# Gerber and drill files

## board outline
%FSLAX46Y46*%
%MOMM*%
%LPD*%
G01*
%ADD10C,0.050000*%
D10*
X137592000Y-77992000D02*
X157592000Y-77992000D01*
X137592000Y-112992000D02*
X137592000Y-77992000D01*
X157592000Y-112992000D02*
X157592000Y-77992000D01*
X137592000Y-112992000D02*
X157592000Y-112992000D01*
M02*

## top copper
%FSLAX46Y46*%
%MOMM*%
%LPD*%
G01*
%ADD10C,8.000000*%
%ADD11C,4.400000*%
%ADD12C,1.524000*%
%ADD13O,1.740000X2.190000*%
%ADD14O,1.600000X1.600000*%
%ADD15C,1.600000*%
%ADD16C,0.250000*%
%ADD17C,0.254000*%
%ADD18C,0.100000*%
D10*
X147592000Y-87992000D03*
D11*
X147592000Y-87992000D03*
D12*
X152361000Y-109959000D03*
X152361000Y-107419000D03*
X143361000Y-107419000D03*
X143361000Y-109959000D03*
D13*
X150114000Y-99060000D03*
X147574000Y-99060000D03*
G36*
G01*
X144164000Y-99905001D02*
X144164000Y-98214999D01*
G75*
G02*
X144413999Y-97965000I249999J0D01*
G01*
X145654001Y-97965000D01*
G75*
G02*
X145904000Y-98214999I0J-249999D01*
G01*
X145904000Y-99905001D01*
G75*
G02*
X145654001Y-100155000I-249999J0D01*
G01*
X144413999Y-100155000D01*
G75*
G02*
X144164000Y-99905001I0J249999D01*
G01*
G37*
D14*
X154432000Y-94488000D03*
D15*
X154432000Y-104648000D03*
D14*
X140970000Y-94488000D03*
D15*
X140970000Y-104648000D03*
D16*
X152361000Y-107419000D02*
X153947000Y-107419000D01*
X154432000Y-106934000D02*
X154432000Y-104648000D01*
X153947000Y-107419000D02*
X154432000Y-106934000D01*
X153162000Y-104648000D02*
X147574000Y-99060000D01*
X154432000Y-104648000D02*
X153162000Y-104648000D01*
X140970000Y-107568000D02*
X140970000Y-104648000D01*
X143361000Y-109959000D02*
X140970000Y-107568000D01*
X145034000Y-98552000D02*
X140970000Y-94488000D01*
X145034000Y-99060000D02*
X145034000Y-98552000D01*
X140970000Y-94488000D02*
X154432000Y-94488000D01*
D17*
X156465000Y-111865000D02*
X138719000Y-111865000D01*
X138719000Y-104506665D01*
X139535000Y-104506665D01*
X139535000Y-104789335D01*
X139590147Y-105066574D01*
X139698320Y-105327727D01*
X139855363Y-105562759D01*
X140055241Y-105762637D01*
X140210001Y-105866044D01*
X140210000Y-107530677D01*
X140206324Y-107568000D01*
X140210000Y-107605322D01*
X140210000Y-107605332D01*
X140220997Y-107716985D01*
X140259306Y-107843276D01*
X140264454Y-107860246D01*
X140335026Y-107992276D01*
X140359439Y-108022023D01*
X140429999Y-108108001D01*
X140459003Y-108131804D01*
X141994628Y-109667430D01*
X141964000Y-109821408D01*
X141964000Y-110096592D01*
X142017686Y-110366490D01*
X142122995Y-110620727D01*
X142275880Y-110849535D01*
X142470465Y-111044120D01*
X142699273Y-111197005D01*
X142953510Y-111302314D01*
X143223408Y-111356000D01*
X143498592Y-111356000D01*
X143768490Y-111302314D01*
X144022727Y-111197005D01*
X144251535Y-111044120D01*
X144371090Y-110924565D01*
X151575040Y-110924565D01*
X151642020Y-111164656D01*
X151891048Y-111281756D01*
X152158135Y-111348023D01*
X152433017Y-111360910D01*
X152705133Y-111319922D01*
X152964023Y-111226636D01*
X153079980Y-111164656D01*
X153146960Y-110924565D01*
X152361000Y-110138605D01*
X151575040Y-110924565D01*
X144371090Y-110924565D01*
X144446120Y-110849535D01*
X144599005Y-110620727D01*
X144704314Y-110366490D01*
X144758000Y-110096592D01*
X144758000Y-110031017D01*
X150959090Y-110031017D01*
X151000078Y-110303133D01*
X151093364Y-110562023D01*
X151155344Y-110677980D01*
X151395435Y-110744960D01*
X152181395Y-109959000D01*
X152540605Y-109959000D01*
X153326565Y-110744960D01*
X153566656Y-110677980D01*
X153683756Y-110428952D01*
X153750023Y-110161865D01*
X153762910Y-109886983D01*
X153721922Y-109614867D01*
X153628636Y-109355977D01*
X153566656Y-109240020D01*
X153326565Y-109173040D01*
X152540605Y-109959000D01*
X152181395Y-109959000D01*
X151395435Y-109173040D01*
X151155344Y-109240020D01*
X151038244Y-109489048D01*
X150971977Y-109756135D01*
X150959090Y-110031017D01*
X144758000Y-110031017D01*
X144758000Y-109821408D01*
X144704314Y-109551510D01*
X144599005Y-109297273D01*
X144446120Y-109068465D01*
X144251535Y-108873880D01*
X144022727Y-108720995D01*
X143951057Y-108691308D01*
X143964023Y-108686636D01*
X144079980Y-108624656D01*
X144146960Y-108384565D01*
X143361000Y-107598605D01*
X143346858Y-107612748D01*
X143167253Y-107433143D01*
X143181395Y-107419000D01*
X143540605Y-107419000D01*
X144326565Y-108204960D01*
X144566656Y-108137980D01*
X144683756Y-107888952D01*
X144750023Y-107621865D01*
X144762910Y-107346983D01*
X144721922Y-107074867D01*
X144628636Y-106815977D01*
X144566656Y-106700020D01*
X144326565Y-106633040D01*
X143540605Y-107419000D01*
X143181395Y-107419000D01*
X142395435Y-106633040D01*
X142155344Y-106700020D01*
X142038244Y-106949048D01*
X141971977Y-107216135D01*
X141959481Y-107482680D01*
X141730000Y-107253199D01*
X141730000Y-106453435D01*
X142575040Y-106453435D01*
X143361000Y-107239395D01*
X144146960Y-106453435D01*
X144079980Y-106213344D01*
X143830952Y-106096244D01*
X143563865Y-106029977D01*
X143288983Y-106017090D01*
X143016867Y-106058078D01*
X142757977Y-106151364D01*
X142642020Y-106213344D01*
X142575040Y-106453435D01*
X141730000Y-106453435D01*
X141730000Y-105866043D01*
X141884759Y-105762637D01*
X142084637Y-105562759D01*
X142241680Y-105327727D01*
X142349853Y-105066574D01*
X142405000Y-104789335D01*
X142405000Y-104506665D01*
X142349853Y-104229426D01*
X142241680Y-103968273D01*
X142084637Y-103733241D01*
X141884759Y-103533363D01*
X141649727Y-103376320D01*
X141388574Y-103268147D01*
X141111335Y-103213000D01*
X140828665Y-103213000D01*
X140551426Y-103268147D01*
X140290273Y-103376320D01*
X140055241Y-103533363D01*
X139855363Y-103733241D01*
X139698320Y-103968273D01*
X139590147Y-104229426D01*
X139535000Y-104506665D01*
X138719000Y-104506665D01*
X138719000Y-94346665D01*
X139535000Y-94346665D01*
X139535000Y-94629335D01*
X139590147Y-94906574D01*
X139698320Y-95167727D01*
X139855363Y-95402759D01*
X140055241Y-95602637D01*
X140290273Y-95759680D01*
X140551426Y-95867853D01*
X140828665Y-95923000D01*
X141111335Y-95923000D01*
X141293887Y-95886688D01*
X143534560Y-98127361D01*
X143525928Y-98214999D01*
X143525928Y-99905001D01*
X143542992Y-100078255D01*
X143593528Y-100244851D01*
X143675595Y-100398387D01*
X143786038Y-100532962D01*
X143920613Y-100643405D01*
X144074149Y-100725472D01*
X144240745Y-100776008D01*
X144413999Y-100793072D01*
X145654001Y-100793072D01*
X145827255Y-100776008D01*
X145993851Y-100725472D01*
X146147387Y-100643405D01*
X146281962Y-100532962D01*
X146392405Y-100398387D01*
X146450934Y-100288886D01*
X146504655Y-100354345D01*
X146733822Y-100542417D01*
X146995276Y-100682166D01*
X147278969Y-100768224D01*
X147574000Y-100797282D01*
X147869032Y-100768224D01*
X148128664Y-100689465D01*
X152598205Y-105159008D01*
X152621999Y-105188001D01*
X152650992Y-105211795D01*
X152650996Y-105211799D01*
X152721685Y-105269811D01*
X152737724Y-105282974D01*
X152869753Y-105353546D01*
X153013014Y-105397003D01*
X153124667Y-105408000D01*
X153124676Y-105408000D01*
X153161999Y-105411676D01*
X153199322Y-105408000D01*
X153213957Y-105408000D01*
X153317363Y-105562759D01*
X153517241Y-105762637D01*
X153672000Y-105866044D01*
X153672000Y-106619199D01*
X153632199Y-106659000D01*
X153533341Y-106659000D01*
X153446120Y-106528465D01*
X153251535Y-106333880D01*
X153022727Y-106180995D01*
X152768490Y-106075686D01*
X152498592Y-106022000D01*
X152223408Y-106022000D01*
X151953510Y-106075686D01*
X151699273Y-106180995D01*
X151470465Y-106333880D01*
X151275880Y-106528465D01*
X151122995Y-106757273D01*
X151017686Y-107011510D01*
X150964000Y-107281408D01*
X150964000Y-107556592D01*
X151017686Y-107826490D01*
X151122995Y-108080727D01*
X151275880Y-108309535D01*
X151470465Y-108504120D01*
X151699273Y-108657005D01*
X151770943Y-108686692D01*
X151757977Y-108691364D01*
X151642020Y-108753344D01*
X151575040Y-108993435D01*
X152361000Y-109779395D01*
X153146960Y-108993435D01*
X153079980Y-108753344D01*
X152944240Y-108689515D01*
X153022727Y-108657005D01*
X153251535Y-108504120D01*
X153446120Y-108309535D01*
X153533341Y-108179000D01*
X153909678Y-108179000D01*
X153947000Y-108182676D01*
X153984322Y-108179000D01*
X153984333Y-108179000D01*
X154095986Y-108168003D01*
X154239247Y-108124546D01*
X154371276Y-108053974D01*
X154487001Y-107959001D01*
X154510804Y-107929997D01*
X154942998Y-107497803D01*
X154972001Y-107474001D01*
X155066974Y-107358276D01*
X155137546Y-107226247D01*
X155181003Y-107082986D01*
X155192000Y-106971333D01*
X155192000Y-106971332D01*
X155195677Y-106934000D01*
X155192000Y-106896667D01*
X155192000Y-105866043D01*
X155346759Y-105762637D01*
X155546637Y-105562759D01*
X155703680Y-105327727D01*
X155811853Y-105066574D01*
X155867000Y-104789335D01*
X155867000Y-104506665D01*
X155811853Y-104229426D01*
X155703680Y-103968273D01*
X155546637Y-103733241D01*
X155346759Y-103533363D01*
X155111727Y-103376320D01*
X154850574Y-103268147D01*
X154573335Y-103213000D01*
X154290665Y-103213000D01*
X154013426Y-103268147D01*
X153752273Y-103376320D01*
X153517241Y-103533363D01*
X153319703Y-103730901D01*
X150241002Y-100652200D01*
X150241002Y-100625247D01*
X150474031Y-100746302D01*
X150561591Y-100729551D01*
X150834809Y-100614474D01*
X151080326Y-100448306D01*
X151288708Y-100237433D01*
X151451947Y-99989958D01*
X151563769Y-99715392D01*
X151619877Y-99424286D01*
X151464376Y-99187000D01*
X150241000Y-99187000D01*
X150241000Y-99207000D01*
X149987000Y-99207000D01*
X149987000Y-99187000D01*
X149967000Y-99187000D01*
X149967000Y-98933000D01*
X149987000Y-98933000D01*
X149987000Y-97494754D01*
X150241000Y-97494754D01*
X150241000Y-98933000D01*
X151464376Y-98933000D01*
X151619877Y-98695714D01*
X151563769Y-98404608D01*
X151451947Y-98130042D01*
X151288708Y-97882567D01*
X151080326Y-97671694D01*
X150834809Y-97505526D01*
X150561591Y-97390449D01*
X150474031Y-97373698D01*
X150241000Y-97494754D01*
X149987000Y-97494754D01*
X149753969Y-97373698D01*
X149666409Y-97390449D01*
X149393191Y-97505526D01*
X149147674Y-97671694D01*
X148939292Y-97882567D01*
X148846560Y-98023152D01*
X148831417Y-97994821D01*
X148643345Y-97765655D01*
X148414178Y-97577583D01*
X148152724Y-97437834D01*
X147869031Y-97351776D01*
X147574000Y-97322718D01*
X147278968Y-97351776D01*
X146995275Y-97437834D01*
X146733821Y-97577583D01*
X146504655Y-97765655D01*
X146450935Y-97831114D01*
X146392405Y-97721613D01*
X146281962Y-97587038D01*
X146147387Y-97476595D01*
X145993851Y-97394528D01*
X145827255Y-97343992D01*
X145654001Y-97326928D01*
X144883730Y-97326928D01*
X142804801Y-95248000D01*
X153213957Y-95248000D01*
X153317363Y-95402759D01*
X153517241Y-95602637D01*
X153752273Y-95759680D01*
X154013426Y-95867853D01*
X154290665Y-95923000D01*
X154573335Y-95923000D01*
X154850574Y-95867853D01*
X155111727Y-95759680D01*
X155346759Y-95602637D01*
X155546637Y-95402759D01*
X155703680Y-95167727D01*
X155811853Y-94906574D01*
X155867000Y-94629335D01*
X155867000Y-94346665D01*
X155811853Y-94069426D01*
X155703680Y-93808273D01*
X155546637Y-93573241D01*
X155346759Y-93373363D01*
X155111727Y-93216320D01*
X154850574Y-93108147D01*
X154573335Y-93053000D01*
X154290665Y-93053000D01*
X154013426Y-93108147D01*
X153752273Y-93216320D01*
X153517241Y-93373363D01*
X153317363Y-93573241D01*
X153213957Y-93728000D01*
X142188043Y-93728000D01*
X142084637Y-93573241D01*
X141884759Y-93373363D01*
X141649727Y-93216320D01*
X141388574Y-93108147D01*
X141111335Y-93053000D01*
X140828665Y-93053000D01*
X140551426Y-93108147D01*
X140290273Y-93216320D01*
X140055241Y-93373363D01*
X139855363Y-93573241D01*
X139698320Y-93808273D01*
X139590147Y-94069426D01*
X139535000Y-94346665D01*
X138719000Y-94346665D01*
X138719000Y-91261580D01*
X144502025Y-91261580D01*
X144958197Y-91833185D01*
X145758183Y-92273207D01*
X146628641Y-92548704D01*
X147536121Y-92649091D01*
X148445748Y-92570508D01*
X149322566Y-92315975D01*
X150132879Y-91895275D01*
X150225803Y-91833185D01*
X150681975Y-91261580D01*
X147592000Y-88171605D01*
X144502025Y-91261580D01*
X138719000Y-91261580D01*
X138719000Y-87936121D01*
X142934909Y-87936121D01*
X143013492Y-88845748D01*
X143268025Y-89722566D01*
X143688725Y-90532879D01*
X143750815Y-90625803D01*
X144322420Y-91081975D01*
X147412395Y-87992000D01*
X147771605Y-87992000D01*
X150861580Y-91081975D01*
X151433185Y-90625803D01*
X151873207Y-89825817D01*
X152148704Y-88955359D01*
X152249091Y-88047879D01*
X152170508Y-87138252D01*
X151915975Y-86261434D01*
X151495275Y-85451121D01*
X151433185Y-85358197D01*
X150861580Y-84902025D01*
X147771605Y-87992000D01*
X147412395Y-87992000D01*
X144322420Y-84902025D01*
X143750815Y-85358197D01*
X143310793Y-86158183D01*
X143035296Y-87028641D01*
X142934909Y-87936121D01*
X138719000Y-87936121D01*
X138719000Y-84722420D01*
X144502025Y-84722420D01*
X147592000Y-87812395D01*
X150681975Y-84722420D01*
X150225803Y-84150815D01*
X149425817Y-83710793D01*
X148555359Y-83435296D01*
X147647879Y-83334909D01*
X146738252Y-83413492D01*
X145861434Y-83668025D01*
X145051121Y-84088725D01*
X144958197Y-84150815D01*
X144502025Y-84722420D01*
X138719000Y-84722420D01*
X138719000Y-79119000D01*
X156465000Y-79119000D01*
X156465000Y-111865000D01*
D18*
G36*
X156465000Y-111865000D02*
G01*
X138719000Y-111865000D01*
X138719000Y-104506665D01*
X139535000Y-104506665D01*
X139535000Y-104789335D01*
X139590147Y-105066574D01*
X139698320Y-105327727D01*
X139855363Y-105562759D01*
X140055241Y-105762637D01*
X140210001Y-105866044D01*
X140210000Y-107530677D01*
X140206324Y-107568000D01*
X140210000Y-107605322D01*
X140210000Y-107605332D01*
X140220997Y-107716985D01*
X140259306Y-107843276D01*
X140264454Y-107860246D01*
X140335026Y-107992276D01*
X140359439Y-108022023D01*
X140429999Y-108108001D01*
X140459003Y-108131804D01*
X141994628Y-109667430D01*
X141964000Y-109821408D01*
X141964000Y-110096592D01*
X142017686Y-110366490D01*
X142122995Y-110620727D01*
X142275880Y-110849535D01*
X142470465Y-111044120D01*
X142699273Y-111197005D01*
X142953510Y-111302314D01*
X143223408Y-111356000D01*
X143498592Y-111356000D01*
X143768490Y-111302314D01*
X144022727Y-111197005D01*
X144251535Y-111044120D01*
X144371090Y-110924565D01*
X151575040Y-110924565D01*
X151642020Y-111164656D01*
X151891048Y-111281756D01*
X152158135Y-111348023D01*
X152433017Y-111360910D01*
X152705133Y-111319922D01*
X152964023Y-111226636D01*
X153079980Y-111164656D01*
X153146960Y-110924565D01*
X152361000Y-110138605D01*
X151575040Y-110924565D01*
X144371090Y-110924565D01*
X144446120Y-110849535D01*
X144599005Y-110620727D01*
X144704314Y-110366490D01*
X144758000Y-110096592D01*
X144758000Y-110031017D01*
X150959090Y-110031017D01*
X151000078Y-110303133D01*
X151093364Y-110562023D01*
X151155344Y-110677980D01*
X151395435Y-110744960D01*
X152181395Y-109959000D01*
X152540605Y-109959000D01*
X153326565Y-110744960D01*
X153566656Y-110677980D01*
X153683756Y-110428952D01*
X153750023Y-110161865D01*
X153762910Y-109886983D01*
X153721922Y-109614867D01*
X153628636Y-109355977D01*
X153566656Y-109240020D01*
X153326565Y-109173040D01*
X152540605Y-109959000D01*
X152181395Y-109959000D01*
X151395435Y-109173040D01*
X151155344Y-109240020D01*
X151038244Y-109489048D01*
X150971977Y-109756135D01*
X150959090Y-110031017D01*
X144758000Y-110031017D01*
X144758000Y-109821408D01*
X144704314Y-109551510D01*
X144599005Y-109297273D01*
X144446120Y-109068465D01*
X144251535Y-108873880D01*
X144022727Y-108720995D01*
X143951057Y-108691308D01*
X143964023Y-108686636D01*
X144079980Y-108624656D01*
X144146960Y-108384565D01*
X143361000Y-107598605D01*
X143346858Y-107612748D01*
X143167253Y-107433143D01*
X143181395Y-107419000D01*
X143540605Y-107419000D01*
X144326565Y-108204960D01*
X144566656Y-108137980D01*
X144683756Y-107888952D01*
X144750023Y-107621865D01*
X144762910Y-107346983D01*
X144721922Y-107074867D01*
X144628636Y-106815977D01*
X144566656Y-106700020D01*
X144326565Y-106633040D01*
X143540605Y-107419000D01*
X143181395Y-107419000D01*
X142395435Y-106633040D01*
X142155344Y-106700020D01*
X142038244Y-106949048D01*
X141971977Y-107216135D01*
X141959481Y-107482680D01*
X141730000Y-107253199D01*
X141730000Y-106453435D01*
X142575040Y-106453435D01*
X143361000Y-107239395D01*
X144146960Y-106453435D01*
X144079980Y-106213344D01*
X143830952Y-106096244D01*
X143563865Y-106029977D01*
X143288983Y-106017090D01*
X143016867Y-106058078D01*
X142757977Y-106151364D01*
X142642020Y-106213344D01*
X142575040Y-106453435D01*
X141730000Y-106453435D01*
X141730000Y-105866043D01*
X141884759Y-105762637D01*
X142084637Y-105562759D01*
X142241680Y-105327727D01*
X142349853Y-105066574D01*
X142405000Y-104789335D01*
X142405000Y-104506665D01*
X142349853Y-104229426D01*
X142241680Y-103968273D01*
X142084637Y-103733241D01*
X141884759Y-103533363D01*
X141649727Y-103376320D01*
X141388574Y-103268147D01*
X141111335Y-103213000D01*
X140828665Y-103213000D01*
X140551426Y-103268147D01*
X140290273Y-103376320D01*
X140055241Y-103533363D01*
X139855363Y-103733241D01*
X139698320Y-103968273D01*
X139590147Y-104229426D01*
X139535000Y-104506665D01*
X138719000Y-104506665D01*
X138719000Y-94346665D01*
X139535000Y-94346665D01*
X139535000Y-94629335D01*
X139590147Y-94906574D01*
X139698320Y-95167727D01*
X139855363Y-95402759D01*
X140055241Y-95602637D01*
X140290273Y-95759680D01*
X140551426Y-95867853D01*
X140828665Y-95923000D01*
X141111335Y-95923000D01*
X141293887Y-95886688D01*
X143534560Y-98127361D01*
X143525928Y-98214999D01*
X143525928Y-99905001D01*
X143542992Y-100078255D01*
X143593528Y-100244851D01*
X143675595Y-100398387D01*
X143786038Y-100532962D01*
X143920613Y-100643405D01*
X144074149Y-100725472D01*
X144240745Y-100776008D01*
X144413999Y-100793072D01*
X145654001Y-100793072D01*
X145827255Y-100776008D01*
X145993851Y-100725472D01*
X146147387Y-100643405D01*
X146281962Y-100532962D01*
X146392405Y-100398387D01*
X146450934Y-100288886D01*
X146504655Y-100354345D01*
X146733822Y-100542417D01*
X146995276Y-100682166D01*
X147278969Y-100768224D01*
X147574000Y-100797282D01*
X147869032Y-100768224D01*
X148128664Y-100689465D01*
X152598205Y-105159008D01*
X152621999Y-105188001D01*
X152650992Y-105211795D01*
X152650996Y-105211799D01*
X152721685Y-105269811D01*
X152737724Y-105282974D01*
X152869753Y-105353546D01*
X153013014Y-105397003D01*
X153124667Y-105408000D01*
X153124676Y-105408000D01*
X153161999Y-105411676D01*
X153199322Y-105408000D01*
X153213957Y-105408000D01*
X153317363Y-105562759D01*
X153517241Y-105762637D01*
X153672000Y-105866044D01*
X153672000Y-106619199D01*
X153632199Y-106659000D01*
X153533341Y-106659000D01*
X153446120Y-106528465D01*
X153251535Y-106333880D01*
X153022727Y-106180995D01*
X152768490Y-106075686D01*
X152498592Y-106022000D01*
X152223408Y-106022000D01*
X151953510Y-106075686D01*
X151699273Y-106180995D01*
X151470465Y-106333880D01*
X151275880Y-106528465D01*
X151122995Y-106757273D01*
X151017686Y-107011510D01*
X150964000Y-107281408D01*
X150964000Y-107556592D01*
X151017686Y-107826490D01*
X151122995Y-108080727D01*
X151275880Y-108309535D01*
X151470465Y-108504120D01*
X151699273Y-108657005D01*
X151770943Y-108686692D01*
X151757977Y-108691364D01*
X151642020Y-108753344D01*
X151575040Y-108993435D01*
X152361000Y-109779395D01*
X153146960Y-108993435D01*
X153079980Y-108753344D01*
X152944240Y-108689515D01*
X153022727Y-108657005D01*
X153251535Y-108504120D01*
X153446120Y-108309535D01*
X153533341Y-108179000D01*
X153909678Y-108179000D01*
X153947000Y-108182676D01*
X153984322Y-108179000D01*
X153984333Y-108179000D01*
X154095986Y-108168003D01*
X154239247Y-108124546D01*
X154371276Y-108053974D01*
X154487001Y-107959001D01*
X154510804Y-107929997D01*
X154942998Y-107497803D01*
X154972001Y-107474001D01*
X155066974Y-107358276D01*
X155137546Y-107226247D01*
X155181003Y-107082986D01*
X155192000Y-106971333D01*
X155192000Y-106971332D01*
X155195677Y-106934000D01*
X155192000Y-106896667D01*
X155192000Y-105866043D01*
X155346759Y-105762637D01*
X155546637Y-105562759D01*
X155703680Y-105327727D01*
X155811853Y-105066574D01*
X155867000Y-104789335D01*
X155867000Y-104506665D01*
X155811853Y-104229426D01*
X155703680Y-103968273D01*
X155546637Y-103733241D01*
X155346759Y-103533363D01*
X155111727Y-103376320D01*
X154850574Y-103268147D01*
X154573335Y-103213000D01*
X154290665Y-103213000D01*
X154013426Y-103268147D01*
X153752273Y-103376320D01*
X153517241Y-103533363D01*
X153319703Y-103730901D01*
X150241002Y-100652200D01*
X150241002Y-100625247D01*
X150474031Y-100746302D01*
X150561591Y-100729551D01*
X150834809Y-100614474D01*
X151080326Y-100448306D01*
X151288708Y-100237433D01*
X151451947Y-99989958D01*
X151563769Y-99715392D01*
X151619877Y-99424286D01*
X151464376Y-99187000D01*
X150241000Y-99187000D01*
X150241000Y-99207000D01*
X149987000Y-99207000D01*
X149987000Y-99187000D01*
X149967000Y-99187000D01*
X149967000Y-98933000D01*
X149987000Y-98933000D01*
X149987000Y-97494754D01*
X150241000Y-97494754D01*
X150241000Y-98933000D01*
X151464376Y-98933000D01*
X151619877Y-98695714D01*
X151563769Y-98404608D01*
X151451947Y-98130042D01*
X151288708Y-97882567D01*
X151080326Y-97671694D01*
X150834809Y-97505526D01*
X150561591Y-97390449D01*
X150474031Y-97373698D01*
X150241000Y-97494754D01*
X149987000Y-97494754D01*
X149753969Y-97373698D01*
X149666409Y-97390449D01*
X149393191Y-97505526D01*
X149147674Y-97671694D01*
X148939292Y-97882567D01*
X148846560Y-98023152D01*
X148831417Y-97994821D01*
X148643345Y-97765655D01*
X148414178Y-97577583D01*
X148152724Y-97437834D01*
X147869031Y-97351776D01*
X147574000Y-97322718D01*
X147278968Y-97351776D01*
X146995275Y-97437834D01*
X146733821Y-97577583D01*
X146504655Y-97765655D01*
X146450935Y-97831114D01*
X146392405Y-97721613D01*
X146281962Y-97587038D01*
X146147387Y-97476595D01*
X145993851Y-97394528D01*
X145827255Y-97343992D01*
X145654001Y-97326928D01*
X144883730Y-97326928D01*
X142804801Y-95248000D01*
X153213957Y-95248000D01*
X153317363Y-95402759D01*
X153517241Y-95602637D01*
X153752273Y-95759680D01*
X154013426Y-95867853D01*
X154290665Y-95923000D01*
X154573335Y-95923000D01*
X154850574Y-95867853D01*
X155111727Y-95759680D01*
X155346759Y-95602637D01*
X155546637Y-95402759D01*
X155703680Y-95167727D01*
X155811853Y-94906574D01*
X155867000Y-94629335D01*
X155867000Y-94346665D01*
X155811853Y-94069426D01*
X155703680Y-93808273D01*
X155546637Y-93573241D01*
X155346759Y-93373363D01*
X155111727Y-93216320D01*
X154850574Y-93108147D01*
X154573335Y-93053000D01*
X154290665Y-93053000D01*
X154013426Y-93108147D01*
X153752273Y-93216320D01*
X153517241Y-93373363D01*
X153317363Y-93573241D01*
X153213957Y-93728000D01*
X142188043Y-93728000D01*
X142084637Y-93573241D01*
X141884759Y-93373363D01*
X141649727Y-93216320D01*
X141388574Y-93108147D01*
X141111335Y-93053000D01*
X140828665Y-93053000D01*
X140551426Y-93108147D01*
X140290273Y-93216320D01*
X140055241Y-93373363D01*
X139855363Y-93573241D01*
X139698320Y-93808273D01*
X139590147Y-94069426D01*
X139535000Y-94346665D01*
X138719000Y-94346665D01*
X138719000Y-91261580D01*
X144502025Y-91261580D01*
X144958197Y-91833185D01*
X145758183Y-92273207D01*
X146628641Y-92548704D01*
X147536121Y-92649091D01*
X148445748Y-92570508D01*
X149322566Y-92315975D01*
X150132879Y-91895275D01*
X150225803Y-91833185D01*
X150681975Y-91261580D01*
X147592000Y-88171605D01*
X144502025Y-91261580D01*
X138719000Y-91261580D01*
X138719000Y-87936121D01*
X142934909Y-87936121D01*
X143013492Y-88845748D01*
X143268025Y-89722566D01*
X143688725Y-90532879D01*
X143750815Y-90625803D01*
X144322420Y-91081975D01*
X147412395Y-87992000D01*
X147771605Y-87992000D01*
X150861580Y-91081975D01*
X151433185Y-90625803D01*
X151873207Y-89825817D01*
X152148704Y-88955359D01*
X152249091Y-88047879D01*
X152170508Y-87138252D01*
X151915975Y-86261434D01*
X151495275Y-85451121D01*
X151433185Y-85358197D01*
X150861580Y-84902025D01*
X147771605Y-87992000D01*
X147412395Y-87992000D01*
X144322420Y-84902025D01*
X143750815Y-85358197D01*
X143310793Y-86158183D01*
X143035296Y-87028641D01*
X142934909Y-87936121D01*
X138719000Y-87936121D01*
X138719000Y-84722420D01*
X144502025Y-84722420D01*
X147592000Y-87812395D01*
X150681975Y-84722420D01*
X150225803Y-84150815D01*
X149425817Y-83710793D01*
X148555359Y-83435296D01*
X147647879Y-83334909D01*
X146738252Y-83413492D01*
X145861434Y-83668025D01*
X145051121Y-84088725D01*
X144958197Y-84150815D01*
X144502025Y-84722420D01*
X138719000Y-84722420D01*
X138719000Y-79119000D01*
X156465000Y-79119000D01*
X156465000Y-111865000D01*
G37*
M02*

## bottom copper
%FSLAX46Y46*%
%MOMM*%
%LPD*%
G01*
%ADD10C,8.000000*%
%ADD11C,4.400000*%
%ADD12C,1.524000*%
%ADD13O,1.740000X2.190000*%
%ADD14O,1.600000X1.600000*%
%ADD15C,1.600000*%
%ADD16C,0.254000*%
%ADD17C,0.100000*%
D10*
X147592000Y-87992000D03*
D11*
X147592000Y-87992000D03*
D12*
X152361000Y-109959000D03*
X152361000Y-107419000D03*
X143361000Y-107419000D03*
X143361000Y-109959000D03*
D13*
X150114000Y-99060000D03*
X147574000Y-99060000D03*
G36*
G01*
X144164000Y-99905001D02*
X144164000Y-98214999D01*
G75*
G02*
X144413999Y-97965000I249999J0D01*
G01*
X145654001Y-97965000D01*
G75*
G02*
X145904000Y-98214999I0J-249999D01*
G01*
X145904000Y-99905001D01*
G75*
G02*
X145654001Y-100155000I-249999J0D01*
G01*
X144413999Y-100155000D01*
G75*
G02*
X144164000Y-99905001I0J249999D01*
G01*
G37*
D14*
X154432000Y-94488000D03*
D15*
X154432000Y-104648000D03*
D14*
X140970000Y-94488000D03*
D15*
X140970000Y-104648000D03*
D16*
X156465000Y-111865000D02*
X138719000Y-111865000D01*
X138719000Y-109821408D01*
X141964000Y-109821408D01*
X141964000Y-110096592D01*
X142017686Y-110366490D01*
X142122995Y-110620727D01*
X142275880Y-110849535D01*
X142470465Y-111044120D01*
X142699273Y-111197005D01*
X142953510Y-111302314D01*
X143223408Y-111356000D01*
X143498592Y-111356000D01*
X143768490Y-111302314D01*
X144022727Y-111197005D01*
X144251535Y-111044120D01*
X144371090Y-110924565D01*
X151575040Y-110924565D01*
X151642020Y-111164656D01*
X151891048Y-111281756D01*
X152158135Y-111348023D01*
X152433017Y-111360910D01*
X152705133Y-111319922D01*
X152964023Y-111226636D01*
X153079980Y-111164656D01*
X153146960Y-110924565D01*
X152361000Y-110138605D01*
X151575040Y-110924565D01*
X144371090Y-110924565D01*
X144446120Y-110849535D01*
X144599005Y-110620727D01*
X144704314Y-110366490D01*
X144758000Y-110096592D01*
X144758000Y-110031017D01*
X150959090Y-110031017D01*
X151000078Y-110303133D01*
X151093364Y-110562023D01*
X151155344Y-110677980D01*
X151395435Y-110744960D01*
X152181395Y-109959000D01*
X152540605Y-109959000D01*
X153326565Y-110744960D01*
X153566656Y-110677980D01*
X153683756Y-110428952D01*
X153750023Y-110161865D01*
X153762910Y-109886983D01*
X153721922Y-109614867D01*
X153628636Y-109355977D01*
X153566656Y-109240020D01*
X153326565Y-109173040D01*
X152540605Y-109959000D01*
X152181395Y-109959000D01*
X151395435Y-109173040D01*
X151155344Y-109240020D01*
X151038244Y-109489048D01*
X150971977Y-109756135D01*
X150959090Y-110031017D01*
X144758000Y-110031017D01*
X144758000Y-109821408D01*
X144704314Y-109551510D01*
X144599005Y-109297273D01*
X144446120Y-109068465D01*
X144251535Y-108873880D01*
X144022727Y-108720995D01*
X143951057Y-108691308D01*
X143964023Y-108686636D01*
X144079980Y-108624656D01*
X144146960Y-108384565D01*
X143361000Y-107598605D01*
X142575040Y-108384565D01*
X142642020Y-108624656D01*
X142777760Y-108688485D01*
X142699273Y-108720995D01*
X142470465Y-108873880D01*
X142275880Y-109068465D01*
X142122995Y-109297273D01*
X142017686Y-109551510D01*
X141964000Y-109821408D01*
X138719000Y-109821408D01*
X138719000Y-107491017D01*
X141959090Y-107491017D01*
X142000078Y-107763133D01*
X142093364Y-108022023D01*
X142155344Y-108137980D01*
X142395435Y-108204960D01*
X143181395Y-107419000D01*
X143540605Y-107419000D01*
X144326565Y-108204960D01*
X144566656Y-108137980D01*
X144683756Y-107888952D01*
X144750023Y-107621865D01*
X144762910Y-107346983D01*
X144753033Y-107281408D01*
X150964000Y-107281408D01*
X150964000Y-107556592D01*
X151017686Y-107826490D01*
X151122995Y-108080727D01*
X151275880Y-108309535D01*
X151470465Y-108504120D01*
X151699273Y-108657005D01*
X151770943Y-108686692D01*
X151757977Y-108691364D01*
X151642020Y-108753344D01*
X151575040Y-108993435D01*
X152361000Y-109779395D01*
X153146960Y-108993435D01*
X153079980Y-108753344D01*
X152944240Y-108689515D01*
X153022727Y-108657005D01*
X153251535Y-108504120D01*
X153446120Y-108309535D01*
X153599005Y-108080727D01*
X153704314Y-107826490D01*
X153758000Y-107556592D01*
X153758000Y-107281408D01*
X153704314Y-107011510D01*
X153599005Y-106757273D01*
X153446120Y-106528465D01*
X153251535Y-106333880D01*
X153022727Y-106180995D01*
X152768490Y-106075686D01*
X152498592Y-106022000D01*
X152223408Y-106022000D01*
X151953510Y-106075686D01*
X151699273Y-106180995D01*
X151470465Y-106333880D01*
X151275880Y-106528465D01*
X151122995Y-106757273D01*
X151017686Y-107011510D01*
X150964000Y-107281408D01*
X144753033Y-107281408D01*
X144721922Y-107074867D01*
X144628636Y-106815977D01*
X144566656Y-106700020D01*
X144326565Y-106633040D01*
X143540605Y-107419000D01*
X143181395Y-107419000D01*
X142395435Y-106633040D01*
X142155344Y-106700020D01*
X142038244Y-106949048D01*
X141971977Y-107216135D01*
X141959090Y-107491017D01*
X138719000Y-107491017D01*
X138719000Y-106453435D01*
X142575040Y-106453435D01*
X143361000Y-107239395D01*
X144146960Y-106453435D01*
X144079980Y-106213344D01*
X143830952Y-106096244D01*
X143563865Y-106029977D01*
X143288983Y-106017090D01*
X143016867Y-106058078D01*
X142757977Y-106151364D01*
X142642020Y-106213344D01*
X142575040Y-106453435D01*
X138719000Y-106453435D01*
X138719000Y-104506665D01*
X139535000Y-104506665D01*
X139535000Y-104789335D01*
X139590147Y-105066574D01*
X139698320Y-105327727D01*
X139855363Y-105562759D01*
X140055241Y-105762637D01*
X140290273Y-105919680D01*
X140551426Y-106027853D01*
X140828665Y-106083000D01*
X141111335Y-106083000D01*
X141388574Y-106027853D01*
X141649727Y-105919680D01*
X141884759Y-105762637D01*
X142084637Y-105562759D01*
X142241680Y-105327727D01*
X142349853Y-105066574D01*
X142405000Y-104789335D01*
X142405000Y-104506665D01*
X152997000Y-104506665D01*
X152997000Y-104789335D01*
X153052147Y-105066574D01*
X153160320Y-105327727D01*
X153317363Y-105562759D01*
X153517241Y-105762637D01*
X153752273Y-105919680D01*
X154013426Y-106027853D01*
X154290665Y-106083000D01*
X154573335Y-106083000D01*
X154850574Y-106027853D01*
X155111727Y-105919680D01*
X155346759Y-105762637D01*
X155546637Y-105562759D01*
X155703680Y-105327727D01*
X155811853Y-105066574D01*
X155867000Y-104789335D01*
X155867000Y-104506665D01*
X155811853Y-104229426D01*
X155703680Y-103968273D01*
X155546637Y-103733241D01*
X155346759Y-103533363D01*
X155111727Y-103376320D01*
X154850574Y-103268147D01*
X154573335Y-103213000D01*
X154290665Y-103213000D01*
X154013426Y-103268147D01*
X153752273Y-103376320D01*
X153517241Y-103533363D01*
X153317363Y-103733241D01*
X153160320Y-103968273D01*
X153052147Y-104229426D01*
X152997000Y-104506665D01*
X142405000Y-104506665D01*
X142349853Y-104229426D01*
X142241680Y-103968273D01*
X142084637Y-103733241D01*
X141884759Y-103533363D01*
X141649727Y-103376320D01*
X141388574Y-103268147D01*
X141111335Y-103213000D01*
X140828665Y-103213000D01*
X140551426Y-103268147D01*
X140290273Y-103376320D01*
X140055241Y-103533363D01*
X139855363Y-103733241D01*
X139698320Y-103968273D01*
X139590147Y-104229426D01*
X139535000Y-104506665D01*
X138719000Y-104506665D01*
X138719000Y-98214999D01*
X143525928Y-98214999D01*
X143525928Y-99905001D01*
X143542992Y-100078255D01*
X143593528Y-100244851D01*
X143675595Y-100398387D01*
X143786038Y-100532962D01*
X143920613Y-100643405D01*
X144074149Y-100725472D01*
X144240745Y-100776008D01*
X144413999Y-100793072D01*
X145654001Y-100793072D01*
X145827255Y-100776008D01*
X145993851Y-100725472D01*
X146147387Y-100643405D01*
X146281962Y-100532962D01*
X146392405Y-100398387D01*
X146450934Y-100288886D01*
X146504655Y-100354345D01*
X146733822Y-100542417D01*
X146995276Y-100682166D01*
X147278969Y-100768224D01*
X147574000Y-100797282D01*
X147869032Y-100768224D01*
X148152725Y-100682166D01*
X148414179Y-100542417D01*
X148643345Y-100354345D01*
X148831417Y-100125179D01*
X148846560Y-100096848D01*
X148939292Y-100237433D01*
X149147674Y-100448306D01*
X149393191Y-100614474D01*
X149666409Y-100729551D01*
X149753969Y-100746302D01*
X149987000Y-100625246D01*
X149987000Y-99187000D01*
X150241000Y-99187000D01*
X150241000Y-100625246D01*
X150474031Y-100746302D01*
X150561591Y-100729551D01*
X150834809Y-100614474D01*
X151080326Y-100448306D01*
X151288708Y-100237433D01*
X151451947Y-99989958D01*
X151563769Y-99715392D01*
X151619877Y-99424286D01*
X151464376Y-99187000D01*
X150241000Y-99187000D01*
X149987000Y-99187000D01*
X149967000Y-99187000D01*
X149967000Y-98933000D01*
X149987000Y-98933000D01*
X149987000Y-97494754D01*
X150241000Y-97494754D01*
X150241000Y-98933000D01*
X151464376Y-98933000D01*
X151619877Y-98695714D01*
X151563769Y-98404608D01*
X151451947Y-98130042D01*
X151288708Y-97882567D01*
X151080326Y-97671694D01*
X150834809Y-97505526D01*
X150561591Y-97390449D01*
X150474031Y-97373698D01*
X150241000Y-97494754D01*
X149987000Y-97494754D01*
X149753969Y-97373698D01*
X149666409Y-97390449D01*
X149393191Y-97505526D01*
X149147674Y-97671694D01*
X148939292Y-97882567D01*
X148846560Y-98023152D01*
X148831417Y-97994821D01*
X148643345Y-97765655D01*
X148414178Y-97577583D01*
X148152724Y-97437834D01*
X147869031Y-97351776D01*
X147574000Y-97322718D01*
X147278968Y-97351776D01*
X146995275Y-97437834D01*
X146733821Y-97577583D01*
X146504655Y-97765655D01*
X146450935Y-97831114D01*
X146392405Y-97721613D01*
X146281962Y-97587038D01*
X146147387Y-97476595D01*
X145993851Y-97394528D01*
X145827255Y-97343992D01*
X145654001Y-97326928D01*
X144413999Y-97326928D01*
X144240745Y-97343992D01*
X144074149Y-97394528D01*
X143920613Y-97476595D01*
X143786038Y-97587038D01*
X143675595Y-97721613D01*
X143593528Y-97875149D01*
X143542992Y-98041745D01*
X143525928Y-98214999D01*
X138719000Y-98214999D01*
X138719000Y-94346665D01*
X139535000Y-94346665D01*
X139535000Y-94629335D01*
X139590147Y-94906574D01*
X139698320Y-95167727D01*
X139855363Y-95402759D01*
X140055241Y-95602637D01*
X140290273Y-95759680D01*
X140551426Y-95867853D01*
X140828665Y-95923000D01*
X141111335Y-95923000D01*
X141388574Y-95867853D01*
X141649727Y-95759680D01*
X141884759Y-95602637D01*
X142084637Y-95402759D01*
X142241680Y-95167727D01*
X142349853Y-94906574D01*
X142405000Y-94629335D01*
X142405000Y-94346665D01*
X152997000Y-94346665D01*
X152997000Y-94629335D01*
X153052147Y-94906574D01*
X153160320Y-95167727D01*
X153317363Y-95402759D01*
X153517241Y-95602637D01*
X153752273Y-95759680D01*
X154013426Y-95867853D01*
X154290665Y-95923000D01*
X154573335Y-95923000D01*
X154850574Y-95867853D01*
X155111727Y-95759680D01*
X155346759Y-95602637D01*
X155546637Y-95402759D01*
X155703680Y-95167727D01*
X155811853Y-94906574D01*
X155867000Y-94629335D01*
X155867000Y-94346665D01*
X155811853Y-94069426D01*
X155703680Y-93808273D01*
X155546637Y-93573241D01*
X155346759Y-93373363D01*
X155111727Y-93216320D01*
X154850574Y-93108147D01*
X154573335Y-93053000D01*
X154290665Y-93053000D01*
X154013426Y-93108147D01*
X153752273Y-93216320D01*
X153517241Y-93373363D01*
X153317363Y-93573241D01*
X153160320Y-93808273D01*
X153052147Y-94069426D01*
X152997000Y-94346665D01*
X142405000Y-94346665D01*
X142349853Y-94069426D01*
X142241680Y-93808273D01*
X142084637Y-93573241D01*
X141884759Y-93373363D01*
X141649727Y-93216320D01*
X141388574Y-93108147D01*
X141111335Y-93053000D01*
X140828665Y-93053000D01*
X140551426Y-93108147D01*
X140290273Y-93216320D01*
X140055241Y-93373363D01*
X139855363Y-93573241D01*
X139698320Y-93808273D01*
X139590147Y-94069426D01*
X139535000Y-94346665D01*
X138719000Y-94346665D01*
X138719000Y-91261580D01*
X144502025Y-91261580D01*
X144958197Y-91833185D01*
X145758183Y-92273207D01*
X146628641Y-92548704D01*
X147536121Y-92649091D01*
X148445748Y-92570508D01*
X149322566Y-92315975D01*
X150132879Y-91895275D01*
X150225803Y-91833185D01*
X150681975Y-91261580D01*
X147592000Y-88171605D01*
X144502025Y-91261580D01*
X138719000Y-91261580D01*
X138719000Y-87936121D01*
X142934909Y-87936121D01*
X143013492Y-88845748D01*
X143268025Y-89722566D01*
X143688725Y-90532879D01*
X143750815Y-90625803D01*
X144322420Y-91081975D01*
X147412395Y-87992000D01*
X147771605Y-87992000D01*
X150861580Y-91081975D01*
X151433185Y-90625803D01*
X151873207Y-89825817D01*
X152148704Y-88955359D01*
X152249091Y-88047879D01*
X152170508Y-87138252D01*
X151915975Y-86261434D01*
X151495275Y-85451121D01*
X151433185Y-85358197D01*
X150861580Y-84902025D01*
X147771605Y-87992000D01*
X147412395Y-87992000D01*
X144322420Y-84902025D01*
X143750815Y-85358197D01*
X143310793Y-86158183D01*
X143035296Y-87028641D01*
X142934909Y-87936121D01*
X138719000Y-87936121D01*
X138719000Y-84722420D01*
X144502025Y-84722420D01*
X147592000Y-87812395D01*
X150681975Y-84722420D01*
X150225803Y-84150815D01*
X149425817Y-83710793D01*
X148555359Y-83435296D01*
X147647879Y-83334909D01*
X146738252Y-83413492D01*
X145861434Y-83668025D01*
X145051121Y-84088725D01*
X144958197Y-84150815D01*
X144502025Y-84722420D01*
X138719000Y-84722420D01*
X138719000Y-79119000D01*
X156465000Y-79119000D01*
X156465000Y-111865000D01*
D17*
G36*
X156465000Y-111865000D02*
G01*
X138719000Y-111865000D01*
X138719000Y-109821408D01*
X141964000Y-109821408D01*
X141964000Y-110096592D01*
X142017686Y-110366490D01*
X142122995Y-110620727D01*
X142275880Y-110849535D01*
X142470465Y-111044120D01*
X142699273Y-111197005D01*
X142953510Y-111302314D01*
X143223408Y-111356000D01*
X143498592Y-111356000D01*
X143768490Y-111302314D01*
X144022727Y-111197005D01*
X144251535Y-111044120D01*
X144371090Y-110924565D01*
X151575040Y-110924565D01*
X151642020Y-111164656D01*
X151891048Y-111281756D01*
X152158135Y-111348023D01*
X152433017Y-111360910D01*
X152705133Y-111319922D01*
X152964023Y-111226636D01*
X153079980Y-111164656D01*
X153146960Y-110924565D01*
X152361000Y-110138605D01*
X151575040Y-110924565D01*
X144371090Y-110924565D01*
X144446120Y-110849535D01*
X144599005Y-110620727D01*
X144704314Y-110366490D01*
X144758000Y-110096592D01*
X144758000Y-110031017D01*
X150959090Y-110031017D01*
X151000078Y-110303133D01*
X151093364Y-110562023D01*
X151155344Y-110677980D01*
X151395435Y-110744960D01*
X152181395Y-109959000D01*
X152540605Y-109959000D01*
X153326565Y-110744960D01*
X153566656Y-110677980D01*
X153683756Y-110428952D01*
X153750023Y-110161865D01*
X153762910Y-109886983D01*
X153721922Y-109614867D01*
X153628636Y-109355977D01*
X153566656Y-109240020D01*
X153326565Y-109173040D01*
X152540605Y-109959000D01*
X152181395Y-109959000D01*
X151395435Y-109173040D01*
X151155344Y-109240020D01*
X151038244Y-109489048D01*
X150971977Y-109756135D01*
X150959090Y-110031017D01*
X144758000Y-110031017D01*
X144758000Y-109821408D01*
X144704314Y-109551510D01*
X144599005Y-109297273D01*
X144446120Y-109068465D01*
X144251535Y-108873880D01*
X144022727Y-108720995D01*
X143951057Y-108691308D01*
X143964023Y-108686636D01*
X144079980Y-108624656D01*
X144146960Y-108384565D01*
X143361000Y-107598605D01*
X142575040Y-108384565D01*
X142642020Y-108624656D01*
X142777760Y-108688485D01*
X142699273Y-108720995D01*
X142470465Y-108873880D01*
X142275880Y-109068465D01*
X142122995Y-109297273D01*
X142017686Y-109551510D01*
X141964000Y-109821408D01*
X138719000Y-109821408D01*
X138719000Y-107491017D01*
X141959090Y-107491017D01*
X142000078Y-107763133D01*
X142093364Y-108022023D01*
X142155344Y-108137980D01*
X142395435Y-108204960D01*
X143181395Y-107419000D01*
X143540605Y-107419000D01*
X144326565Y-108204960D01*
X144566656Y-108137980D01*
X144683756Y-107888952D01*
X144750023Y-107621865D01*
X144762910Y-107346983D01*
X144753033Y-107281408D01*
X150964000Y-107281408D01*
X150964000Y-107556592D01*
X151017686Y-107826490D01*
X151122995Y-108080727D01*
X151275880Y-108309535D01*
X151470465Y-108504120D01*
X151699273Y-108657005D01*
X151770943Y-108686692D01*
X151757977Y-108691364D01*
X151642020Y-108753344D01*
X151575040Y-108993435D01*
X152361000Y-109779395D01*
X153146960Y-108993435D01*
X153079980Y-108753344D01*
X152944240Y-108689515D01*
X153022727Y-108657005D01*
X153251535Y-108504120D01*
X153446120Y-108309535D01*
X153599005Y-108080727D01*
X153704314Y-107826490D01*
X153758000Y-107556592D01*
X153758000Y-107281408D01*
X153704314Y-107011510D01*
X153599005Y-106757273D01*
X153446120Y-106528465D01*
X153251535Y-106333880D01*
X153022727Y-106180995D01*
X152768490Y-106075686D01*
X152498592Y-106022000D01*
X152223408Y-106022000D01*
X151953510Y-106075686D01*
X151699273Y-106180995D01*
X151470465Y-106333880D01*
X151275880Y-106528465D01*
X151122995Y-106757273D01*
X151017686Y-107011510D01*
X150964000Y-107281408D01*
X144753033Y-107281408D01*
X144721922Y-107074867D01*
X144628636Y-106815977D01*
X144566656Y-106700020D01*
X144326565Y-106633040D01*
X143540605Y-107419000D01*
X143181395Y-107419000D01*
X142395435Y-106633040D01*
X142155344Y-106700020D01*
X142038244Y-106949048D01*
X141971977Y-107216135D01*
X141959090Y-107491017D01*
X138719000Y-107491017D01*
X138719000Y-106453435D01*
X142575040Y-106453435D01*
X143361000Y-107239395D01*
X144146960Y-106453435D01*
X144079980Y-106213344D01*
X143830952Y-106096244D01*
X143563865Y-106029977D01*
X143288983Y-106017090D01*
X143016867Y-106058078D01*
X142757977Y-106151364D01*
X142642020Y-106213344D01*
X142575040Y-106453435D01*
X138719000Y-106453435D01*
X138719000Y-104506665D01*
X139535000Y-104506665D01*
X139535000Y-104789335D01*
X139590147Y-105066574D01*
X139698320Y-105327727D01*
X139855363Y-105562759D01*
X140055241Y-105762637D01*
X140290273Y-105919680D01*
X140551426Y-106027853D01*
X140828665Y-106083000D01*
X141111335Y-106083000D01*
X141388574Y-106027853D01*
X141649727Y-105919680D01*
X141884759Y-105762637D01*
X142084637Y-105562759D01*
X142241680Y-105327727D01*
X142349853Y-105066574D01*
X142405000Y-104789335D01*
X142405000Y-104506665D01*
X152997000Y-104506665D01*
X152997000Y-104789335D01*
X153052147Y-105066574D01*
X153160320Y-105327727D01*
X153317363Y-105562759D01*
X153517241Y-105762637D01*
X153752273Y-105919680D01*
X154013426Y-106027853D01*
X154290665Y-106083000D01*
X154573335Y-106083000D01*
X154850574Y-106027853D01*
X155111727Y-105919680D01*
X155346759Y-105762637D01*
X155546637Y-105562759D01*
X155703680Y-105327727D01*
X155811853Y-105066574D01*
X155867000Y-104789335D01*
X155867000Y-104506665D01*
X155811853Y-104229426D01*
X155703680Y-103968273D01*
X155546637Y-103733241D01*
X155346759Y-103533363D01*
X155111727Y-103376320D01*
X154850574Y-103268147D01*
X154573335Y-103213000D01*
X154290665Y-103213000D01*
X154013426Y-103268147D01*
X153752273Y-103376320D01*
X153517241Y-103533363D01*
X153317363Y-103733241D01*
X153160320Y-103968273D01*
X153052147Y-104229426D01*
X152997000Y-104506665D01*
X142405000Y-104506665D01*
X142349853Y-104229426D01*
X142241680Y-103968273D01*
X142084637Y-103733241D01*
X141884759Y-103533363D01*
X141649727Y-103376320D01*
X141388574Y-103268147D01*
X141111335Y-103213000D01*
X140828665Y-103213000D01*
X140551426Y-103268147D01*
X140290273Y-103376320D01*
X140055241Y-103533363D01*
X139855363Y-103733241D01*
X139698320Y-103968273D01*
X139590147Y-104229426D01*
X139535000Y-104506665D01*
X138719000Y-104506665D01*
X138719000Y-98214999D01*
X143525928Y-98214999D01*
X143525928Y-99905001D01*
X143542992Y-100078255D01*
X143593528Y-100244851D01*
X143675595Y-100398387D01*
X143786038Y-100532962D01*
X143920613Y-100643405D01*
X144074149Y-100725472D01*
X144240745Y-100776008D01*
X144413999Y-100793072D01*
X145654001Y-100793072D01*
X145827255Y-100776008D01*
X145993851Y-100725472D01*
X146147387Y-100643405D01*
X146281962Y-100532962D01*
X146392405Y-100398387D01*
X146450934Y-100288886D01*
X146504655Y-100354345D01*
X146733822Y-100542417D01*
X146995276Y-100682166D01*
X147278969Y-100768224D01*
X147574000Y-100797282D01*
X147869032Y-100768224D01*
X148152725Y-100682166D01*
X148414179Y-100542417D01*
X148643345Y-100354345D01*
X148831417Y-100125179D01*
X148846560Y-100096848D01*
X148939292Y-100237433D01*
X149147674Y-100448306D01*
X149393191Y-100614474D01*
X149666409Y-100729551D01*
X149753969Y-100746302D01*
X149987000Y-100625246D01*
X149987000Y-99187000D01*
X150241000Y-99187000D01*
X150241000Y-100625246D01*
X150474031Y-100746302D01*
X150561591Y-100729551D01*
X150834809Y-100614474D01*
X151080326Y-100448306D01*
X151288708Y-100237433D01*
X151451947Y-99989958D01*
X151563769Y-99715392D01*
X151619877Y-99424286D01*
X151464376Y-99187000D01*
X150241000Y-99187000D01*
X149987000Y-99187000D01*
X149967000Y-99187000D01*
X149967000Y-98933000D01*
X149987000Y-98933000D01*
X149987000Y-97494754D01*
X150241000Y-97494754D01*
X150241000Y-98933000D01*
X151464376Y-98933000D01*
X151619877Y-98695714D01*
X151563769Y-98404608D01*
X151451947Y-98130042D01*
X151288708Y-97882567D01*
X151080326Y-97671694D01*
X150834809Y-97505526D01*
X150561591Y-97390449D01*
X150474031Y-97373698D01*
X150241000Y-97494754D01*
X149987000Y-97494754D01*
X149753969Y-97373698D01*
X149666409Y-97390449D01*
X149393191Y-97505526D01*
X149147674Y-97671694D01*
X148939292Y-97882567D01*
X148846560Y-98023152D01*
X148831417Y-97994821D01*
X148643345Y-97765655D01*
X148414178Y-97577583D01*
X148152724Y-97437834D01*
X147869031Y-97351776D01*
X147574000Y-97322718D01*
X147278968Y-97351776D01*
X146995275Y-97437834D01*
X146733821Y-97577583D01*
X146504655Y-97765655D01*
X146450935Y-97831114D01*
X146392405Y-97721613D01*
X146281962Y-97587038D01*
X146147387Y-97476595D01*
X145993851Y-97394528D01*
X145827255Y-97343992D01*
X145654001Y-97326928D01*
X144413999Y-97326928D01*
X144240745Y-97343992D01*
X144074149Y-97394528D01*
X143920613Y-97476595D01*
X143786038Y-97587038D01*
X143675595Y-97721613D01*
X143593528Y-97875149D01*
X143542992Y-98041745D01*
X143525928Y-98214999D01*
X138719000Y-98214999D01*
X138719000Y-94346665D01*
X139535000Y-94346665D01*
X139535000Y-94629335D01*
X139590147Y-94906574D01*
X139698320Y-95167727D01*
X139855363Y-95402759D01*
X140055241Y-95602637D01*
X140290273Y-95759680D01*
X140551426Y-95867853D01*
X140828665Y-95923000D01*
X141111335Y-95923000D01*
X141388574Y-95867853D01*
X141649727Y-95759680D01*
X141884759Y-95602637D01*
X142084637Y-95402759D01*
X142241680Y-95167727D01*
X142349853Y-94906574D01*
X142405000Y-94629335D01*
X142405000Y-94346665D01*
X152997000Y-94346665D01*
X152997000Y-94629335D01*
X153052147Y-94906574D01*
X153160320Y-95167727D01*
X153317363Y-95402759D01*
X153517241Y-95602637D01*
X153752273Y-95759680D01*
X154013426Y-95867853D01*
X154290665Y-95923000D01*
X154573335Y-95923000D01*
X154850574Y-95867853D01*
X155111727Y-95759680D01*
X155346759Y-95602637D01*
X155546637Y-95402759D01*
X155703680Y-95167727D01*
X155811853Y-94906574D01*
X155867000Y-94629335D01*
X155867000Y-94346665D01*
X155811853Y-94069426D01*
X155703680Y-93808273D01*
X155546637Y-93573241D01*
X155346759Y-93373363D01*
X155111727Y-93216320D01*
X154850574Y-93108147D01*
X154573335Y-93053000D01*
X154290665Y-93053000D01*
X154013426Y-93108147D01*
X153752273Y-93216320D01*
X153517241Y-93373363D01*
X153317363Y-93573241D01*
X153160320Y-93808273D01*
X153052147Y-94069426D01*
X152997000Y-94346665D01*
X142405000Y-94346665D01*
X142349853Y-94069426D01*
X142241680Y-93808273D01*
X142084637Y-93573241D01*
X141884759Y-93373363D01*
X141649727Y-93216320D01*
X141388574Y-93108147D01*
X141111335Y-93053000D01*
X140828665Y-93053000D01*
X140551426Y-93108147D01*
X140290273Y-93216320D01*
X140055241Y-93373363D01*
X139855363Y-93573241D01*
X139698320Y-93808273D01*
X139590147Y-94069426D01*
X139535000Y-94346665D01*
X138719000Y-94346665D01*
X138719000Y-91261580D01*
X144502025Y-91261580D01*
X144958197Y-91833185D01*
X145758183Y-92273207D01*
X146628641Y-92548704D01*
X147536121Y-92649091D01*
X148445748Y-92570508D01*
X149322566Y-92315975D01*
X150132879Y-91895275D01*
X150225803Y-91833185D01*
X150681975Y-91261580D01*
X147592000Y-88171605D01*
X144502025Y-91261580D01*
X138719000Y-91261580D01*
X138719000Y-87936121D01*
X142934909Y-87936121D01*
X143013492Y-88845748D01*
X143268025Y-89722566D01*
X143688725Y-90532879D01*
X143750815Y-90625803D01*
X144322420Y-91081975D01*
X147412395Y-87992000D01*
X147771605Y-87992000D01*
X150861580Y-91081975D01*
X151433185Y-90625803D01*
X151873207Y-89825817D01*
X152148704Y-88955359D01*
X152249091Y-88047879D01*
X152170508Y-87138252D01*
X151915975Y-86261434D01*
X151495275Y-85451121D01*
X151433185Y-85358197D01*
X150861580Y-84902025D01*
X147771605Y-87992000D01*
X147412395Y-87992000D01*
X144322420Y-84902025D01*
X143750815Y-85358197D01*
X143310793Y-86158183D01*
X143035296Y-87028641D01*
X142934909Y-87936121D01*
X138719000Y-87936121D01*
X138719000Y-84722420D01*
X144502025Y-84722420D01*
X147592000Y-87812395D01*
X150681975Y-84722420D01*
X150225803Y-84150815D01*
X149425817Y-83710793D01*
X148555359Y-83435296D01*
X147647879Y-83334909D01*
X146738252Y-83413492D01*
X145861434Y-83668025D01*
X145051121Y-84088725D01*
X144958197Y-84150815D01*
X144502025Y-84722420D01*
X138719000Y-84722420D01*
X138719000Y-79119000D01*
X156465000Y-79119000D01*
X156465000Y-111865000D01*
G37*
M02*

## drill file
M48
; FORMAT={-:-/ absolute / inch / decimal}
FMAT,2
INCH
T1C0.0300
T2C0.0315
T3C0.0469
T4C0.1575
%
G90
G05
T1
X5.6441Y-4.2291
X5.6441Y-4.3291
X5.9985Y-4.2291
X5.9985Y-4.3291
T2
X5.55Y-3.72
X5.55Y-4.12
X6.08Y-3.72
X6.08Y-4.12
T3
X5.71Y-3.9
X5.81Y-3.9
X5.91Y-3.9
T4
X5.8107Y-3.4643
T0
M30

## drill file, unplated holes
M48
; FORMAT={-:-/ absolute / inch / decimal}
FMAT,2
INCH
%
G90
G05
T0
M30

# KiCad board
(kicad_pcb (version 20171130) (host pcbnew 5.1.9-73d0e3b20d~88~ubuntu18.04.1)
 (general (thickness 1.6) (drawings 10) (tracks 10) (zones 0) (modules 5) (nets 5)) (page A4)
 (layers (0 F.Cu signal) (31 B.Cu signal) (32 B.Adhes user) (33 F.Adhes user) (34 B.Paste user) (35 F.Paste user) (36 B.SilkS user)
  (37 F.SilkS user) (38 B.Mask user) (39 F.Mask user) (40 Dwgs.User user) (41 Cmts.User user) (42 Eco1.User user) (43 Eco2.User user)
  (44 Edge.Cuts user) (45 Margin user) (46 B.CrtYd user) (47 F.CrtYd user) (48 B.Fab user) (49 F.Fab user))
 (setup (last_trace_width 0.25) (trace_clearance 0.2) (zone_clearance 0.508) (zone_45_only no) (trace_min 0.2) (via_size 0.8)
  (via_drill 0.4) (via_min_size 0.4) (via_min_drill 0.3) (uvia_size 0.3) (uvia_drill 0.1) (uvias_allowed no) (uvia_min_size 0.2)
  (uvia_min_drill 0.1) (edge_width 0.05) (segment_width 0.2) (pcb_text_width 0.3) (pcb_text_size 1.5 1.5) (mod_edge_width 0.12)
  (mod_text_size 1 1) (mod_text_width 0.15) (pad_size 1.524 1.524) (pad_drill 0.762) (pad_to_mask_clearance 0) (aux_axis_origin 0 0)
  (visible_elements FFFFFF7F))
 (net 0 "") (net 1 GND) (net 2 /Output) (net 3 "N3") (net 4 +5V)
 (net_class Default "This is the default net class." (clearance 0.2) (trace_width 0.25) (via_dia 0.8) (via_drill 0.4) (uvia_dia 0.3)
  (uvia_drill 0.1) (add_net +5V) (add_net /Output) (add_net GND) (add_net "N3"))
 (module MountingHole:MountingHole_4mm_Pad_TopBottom (layer F.Cu) (at 147.592 87.992)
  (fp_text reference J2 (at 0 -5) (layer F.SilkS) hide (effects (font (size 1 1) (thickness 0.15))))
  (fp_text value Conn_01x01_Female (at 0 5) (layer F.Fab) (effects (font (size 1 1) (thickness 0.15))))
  (pad 1 connect circle (at 0 0) (size 8 8) (layers B.Cu B.Mask) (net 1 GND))
  (pad 1 connect circle (at 0 0) (size 8 8) (layers F.Cu F.Mask) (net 1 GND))
  (pad 1 thru_hole circle (at 0 0) (size 4.4 4.4) (drill 4) (layers *.Cu *.Mask) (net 1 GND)))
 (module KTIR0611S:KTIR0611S (layer B.Cu) (at 147.592 108.792)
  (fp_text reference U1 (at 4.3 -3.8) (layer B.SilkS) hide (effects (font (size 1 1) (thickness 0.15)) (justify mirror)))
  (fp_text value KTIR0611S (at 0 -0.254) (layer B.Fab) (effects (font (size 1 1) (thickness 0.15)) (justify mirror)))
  (pad 4 thru_hole circle (at 4.769 1.167) (size 1.524 1.524) (drill 0.762) (layers *.Cu *.Mask) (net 1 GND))
  (pad 3 thru_hole circle (at 4.769 -1.373) (size 1.524 1.524) (drill 0.762) (layers *.Cu *.Mask) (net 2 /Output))
  (pad 2 thru_hole circle (at -4.231 -1.373) (size 1.524 1.524) (drill 0.762) (layers *.Cu *.Mask) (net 1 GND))
  (pad 1 thru_hole circle (at -4.231 1.167) (size 1.524 1.524) (drill 0.762) (layers *.Cu *.Mask) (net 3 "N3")))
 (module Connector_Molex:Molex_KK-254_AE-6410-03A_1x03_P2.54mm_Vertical (layer F.Cu) (at 145.034 99.06)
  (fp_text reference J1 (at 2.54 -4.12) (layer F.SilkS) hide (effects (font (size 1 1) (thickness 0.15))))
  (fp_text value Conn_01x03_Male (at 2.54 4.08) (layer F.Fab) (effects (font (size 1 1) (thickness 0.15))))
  (pad 3 thru_hole oval (at 5.08 0) (size 1.74 2.19) (drill 1.19) (layers *.Cu *.Mask) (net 1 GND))
  (pad 2 thru_hole oval (at 2.54 0) (size 1.74 2.19) (drill 1.19) (layers *.Cu *.Mask) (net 2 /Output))
  (pad 1 thru_hole roundrect (at 0 0) (size 1.74 2.19) (drill 1.19) (layers *.Cu *.Mask) (roundrect_rratio 0.143678) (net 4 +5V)))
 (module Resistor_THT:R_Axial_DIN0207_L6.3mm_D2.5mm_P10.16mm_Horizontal (layer F.Cu) (at 154.432 104.648 90)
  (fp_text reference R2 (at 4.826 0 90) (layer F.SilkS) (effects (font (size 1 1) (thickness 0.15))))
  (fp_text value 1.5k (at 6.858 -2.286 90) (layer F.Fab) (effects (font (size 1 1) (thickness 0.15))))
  (pad 2 thru_hole oval (at 10.16 0 90) (size 1.6 1.6) (drill 0.8) (layers *.Cu *.Mask) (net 4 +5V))
  (pad 1 thru_hole circle (at 0 0 90) (size 1.6 1.6) (drill 0.8) (layers *.Cu *.Mask) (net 2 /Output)))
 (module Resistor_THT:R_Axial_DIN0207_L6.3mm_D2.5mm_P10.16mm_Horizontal (layer F.Cu) (at 140.97 104.648 90)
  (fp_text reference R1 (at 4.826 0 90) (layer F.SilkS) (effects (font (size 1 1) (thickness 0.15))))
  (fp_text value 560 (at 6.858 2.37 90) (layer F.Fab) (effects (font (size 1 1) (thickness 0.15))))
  (pad 2 thru_hole oval (at 10.16 0 90) (size 1.6 1.6) (drill 0.8) (layers *.Cu *.Mask) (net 4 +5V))
  (pad 1 thru_hole circle (at 0 0 90) (size 1.6 1.6) (drill 0.8) (layers *.Cu *.Mask) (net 3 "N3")))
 (gr_line (start 137.592 77.992) (end 157.592 77.992) (layer Edge.Cuts) (width 0.05))
 (gr_line (start 137.592 112.992) (end 137.592 77.992) (layer Edge.Cuts) (width 0.05))
 (gr_line (start 157.592 112.992) (end 157.592 77.992) (layer Edge.Cuts) (width 0.05))
 (gr_line (start 137.592 112.992) (end 157.592 112.992) (layer Edge.Cuts) (width 0.05))
 (segment (start 152.361 107.419) (end 153.947 107.419) (width 0.25) (layer F.Cu) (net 2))
 (segment (start 154.432 106.934) (end 154.432 104.648) (width 0.25) (layer F.Cu) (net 2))
 (segment (start 153.947 107.419) (end 154.432 106.934) (width 0.25) (layer F.Cu) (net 2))
 (segment (start 153.162 104.648) (end 147.574 99.06) (width 0.25) (layer F.Cu) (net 2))
 (segment (start 154.432 104.648) (end 153.162 104.648) (width 0.25) (layer F.Cu) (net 2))
 (segment (start 140.97 107.568) (end 140.97 104.648) (width 0.25) (layer F.Cu) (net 3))
 (segment (start 143.361 109.959) (end 140.97 107.568) (width 0.25) (layer F.Cu) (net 3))
 (segment (start 145.034 98.552) (end 140.97 94.488) (width 0.25) (layer F.Cu) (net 4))
 (segment (start 145.034 99.06) (end 145.034 98.552) (width 0.25) (layer F.Cu) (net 4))
 (segment (start 140.97 94.488) (end 154.432 94.488) (width 0.25) (layer F.Cu) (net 4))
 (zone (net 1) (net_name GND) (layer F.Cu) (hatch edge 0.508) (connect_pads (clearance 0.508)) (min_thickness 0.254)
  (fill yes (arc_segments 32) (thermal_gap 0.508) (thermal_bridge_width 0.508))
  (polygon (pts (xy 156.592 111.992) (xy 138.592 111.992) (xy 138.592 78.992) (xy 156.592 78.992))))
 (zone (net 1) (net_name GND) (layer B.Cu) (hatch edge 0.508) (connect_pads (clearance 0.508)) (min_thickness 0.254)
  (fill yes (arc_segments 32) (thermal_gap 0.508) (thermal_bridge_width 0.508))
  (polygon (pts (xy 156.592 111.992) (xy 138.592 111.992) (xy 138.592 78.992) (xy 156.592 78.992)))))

